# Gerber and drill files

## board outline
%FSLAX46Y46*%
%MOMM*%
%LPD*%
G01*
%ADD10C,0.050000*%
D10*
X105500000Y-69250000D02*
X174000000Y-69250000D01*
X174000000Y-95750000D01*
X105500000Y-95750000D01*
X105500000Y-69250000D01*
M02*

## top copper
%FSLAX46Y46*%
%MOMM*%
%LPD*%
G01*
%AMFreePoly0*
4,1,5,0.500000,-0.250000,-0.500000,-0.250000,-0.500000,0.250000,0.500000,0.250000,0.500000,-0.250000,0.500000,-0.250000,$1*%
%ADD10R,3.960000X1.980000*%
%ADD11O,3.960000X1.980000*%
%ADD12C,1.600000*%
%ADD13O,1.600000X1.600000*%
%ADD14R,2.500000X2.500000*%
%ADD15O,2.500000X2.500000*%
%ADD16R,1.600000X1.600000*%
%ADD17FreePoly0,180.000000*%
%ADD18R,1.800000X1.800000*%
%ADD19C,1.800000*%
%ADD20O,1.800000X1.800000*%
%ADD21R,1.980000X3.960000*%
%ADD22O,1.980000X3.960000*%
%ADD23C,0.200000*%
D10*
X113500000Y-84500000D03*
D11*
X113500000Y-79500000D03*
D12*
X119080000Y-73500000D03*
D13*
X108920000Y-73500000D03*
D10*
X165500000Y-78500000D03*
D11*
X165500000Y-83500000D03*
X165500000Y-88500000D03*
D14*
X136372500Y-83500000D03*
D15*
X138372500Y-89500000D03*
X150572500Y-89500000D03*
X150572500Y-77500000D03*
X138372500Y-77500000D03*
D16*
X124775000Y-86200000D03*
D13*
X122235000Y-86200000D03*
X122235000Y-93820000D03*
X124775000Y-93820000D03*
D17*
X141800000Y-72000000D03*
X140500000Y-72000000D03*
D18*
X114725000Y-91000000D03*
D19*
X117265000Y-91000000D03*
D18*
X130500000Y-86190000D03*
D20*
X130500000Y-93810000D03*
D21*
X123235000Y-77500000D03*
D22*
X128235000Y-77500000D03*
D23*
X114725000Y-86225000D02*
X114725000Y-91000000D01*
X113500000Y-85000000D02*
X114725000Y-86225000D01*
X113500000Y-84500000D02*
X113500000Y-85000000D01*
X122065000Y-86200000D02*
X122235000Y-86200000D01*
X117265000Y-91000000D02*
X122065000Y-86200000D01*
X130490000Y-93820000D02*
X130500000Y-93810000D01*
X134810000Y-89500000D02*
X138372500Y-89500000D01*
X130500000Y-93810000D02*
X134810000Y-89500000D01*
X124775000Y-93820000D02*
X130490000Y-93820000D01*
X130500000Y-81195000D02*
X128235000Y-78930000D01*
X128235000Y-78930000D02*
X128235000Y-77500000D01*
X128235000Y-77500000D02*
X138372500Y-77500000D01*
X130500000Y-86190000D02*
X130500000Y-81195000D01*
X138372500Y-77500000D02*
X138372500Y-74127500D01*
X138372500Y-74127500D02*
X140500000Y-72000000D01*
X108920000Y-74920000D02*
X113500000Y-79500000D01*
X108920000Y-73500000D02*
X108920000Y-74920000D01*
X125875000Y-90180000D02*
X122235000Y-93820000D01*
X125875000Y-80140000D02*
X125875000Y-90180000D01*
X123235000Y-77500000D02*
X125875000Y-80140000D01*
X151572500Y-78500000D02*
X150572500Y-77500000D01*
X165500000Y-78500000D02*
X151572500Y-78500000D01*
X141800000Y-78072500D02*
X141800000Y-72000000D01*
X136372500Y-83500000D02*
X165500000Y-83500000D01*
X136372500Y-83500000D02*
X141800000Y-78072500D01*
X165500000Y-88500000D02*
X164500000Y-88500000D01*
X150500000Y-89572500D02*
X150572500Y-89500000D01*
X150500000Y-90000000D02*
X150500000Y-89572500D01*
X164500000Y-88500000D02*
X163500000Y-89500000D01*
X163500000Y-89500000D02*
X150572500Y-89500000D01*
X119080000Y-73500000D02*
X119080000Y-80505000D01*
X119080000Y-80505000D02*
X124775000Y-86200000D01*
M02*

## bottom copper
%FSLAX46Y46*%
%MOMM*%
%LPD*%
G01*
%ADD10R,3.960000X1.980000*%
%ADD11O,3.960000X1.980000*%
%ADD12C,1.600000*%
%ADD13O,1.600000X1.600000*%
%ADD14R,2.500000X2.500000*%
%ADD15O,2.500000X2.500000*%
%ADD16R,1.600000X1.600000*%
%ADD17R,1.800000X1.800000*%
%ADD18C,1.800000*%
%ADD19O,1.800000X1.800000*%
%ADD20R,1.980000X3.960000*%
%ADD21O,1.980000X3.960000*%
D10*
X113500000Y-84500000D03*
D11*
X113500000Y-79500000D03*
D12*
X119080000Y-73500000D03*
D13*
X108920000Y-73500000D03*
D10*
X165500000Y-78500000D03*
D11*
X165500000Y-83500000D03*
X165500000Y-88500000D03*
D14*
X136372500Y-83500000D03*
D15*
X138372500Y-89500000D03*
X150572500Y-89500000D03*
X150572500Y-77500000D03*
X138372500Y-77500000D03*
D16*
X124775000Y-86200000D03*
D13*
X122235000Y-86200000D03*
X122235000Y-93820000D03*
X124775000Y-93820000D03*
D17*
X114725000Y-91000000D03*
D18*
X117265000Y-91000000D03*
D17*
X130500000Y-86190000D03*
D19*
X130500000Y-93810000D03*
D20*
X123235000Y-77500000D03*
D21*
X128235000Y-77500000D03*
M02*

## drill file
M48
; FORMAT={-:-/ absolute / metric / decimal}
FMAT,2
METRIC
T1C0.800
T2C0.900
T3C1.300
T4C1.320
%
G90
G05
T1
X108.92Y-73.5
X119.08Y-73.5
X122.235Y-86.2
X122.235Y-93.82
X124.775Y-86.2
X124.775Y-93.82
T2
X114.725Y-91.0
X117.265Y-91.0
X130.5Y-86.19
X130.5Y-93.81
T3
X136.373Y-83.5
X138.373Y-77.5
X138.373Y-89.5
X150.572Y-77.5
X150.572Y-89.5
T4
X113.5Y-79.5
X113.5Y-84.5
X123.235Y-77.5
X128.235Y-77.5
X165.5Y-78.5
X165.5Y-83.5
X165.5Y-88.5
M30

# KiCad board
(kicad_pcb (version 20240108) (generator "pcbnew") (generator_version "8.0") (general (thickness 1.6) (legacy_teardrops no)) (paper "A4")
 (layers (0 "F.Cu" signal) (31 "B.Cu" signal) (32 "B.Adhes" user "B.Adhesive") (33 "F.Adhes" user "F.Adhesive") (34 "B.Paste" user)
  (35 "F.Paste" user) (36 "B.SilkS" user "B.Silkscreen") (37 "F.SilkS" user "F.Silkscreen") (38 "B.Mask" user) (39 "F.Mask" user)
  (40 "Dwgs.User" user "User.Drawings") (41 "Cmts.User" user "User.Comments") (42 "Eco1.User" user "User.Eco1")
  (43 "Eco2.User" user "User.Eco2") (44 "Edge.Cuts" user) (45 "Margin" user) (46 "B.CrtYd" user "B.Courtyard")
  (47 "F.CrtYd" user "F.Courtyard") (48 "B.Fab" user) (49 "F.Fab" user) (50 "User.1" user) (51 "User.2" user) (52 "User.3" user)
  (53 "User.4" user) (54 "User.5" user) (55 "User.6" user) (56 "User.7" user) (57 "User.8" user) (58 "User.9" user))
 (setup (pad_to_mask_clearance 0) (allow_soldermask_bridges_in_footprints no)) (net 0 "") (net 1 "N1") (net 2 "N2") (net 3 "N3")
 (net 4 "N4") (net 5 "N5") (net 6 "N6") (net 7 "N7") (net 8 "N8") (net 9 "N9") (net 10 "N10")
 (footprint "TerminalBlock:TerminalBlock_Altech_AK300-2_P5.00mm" (layer "F.Cu") (at 113.5 84.5 90)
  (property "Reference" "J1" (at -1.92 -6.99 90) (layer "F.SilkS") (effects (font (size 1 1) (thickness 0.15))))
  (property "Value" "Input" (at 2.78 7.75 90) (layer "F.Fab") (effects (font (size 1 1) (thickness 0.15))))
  (pad "1" thru_hole rect (at 0 0 90) (size 1.98 3.96) (drill 1.32) (layers "*.Cu" "*.Mask") (remove_unused_layers no) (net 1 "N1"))
  (pad "2" thru_hole oval (at 5 0 90) (size 1.98 3.96) (drill 1.32) (layers "*.Cu" "*.Mask") (remove_unused_layers no) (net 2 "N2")))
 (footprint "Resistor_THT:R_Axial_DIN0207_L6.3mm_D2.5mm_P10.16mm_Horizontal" (layer "F.Cu") (at 119.08 73.5 180)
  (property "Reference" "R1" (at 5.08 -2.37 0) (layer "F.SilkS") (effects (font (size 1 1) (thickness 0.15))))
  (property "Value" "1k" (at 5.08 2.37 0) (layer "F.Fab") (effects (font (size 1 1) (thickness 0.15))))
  (pad "1" thru_hole circle (at 0 0 180) (size 1.6 1.6) (drill 0.8) (layers "*.Cu" "*.Mask") (remove_unused_layers no) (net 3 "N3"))
  (pad "2" thru_hole oval (at 10.16 0 180) (size 1.6 1.6) (drill 0.8) (layers "*.Cu" "*.Mask") (remove_unused_layers no) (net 2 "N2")))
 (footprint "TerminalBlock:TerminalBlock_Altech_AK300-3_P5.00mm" (layer "F.Cu") (at 165.5 78.5 -90)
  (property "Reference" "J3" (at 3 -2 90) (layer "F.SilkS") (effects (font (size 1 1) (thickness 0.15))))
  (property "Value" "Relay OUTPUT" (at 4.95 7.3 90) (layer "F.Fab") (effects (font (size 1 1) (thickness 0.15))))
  (pad "1" thru_hole rect (at 0 0 270) (size 1.98 3.96) (drill 1.32) (layers "*.Cu" "*.Mask") (remove_unused_layers no) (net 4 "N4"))
  (pad "2" thru_hole oval (at 5 0 270) (size 1.98 3.96) (drill 1.32) (layers "*.Cu" "*.Mask") (remove_unused_layers no) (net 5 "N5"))
  (pad "3" thru_hole oval (at 10 0 270) (size 1.98 3.96) (drill 1.32) (layers "*.Cu" "*.Mask") (remove_unused_layers no) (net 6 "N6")))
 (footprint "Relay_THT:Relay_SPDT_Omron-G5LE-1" (layer "F.Cu") (at 136.3725 83.5 90)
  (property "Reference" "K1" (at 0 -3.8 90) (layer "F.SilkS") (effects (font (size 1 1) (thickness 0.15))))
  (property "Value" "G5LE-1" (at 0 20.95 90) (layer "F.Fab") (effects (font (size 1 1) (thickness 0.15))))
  (pad "1" thru_hole rect (at 0 0 90) (size 2.5 2.5) (drill 1.3) (layers "*.Cu" "*.Mask") (remove_unused_layers no) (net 5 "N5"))
  (pad "2" thru_hole oval (at -6 2 90) (size 2.5 2.5) (drill 1.3) (layers "*.Cu" "*.Mask") (remove_unused_layers no) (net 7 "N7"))
  (pad "3" thru_hole oval (at -6 14.2 90) (size 2.5 2.5) (drill 1.3) (layers "*.Cu" "*.Mask") (remove_unused_layers no) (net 6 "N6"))
  (pad "4" thru_hole oval (at 6 14.2 90) (size 2.5 2.5) (drill 1.3) (layers "*.Cu" "*.Mask") (remove_unused_layers no) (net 4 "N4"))
  (pad "5" thru_hole oval (at 6 2 90) (size 2.5 2.5) (drill 1.3) (layers "*.Cu" "*.Mask") (remove_unused_layers no) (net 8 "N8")))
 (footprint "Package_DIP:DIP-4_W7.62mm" (layer "F.Cu") (at 124.775 86.2 -90)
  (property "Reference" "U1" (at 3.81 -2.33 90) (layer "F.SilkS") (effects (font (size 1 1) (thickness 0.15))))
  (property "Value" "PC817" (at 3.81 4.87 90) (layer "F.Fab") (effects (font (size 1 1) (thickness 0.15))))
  (pad "1" thru_hole rect (at 0 0 270) (size 1.6 1.6) (drill 0.8) (layers "*.Cu" "*.Mask") (remove_unused_layers no) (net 3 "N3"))
  (pad "2" thru_hole oval (at 0 2.54 270) (size 1.6 1.6) (drill 0.8) (layers "*.Cu" "*.Mask") (remove_unused_layers no) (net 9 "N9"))
  (pad "3" thru_hole oval (at 7.62 2.54 270) (size 1.6 1.6) (drill 0.8) (layers "*.Cu" "*.Mask") (remove_unused_layers no) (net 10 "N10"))
  (pad "4" thru_hole oval (at 7.62 0 270) (size 1.6 1.6) (drill 0.8) (layers "*.Cu" "*.Mask") (remove_unused_layers no) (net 7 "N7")))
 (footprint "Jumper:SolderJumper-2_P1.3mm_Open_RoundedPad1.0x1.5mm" (layer "F.Cu") (at 141.15 72 180)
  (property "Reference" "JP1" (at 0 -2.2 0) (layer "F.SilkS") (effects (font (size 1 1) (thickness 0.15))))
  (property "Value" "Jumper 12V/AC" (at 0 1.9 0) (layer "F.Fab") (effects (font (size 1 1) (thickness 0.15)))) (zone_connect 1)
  (pad "1" smd custom (at -0.65 0 180) (size 1 0.5) (layers "F.Cu" "F.Mask") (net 5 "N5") (zone_connect 2) (thermal_bridge_angle 45)
   (options (clearance outline) (anchor rect)) (primitives))
  (pad "2" smd custom (at 0.65 0 180) (size 1 0.5) (layers "F.Cu" "F.Mask") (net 8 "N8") (zone_connect 2) (thermal_bridge_angle 45)
   (options (clearance outline) (anchor rect)) (primitives)))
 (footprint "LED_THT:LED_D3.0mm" (layer "F.Cu") (at 114.725 91)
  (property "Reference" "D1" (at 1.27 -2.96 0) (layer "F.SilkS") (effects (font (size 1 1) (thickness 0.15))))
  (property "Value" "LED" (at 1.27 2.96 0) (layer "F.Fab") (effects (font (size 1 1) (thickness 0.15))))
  (pad "1" thru_hole rect (at 0 0) (size 1.8 1.8) (drill 0.9) (layers "*.Cu" "*.Mask") (remove_unused_layers no) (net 1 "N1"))
  (pad "2" thru_hole circle (at 2.54 0) (size 1.8 1.8) (drill 0.9) (layers "*.Cu" "*.Mask") (remove_unused_layers no) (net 9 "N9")))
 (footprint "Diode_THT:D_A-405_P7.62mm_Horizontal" (layer "F.Cu") (at 130.5 86.19 -90)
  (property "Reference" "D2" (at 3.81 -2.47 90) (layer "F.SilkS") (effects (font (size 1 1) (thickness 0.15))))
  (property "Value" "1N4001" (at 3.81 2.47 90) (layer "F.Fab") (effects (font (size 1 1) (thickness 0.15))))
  (pad "1" thru_hole rect (at 0 0 270) (size 1.8 1.8) (drill 0.9) (layers "*.Cu" "*.Mask") (remove_unused_layers no) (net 8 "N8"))
  (pad "2" thru_hole oval (at 7.62 0 270) (size 1.8 1.8) (drill 0.9) (layers "*.Cu" "*.Mask") (remove_unused_layers no) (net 7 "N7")))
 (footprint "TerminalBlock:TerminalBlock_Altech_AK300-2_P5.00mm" (layer "F.Cu") (at 123.235 77.5)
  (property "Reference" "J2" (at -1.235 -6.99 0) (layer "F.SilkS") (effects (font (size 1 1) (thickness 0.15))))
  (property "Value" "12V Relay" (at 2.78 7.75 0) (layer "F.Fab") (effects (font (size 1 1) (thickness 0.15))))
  (pad "1" thru_hole rect (at 0 0) (size 1.98 3.96) (drill 1.32) (layers "*.Cu" "*.Mask") (remove_unused_layers no) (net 10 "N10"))
  (pad "2" thru_hole oval (at 5 0) (size 1.98 3.96) (drill 1.32) (layers "*.Cu" "*.Mask") (remove_unused_layers no) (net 8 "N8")))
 (gr_rect (start 105.5 69.25) (end 174 95.75) (stroke (width 0.05) (type default)) (fill none) (layer "Edge.Cuts"))
 (segment (start 114.725 86.225) (end 114.725 91) (width 0.2) (layer "F.Cu") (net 1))
 (segment (start 113.5 85) (end 114.725 86.225) (width 0.2) (layer "F.Cu") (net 1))
 (segment (start 113.5 84.5) (end 113.5 85) (width 0.2) (layer "F.Cu") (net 1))
 (segment (start 122.065 86.2) (end 122.235 86.2) (width 0.2) (layer "F.Cu") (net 9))
 (segment (start 117.265 91) (end 122.065 86.2) (width 0.2) (layer "F.Cu") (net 9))
 (segment (start 130.49 93.82) (end 130.5 93.81) (width 0.2) (layer "F.Cu") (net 7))
 (segment (start 134.81 89.5) (end 138.3725 89.5) (width 0.2) (layer "F.Cu") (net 7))
 (segment (start 130.5 93.81) (end 134.81 89.5) (width 0.2) (layer "F.Cu") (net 7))
 (segment (start 124.775 93.82) (end 130.49 93.82) (width 0.2) (layer "F.Cu") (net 7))
 (segment (start 130.5 81.195) (end 128.235 78.93) (width 0.2) (layer "F.Cu") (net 8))
 (segment (start 128.235 78.93) (end 128.235 77.5) (width 0.2) (layer "F.Cu") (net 8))
 (segment (start 128.235 77.5) (end 138.3725 77.5) (width 0.2) (layer "F.Cu") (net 8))
 (segment (start 130.5 86.19) (end 130.5 81.195) (width 0.2) (layer "F.Cu") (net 8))
 (segment (start 138.3725 77.5) (end 138.3725 74.1275) (width 0.2) (layer "F.Cu") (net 8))
 (segment (start 138.3725 74.1275) (end 140.5 72) (width 0.2) (layer "F.Cu") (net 8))
 (segment (start 108.92 74.92) (end 113.5 79.5) (width 0.2) (layer "F.Cu") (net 2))
 (segment (start 108.92 73.5) (end 108.92 74.92) (width 0.2) (layer "F.Cu") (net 2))
 (segment (start 125.875 90.18) (end 122.235 93.82) (width 0.2) (layer "F.Cu") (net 10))
 (segment (start 125.875 80.14) (end 125.875 90.18) (width 0.2) (layer "F.Cu") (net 10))
 (segment (start 123.235 77.5) (end 125.875 80.14) (width 0.2) (layer "F.Cu") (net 10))
 (segment (start 151.5725 78.5) (end 150.5725 77.5) (width 0.2) (layer "F.Cu") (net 4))
 (segment (start 165.5 78.5) (end 151.5725 78.5) (width 0.2) (layer "F.Cu") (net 4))
 (segment (start 141.8 78.0725) (end 141.8 72) (width 0.2) (layer "F.Cu") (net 5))
 (segment (start 136.3725 83.5) (end 165.5 83.5) (width 0.2) (layer "F.Cu") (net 5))
 (segment (start 136.3725 83.5) (end 141.8 78.0725) (width 0.2) (layer "F.Cu") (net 5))
 (segment (start 165.5 88.5) (end 164.5 88.5) (width 0.2) (layer "F.Cu") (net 6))
 (segment (start 150.5 89.5725) (end 150.5725 89.5) (width 0.2) (layer "F.Cu") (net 6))
 (segment (start 150.5 90) (end 150.5 89.5725) (width 0.2) (layer "F.Cu") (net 6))
 (segment (start 164.5 88.5) (end 163.5 89.5) (width 0.2) (layer "F.Cu") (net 6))
 (segment (start 163.5 89.5) (end 150.5725 89.5) (width 0.2) (layer "F.Cu") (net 6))
 (segment (start 119.08 73.5) (end 119.08 80.505) (width 0.2) (layer "F.Cu") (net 3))
 (segment (start 119.08 80.505) (end 124.775 86.2) (width 0.2) (layer "F.Cu") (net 3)))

